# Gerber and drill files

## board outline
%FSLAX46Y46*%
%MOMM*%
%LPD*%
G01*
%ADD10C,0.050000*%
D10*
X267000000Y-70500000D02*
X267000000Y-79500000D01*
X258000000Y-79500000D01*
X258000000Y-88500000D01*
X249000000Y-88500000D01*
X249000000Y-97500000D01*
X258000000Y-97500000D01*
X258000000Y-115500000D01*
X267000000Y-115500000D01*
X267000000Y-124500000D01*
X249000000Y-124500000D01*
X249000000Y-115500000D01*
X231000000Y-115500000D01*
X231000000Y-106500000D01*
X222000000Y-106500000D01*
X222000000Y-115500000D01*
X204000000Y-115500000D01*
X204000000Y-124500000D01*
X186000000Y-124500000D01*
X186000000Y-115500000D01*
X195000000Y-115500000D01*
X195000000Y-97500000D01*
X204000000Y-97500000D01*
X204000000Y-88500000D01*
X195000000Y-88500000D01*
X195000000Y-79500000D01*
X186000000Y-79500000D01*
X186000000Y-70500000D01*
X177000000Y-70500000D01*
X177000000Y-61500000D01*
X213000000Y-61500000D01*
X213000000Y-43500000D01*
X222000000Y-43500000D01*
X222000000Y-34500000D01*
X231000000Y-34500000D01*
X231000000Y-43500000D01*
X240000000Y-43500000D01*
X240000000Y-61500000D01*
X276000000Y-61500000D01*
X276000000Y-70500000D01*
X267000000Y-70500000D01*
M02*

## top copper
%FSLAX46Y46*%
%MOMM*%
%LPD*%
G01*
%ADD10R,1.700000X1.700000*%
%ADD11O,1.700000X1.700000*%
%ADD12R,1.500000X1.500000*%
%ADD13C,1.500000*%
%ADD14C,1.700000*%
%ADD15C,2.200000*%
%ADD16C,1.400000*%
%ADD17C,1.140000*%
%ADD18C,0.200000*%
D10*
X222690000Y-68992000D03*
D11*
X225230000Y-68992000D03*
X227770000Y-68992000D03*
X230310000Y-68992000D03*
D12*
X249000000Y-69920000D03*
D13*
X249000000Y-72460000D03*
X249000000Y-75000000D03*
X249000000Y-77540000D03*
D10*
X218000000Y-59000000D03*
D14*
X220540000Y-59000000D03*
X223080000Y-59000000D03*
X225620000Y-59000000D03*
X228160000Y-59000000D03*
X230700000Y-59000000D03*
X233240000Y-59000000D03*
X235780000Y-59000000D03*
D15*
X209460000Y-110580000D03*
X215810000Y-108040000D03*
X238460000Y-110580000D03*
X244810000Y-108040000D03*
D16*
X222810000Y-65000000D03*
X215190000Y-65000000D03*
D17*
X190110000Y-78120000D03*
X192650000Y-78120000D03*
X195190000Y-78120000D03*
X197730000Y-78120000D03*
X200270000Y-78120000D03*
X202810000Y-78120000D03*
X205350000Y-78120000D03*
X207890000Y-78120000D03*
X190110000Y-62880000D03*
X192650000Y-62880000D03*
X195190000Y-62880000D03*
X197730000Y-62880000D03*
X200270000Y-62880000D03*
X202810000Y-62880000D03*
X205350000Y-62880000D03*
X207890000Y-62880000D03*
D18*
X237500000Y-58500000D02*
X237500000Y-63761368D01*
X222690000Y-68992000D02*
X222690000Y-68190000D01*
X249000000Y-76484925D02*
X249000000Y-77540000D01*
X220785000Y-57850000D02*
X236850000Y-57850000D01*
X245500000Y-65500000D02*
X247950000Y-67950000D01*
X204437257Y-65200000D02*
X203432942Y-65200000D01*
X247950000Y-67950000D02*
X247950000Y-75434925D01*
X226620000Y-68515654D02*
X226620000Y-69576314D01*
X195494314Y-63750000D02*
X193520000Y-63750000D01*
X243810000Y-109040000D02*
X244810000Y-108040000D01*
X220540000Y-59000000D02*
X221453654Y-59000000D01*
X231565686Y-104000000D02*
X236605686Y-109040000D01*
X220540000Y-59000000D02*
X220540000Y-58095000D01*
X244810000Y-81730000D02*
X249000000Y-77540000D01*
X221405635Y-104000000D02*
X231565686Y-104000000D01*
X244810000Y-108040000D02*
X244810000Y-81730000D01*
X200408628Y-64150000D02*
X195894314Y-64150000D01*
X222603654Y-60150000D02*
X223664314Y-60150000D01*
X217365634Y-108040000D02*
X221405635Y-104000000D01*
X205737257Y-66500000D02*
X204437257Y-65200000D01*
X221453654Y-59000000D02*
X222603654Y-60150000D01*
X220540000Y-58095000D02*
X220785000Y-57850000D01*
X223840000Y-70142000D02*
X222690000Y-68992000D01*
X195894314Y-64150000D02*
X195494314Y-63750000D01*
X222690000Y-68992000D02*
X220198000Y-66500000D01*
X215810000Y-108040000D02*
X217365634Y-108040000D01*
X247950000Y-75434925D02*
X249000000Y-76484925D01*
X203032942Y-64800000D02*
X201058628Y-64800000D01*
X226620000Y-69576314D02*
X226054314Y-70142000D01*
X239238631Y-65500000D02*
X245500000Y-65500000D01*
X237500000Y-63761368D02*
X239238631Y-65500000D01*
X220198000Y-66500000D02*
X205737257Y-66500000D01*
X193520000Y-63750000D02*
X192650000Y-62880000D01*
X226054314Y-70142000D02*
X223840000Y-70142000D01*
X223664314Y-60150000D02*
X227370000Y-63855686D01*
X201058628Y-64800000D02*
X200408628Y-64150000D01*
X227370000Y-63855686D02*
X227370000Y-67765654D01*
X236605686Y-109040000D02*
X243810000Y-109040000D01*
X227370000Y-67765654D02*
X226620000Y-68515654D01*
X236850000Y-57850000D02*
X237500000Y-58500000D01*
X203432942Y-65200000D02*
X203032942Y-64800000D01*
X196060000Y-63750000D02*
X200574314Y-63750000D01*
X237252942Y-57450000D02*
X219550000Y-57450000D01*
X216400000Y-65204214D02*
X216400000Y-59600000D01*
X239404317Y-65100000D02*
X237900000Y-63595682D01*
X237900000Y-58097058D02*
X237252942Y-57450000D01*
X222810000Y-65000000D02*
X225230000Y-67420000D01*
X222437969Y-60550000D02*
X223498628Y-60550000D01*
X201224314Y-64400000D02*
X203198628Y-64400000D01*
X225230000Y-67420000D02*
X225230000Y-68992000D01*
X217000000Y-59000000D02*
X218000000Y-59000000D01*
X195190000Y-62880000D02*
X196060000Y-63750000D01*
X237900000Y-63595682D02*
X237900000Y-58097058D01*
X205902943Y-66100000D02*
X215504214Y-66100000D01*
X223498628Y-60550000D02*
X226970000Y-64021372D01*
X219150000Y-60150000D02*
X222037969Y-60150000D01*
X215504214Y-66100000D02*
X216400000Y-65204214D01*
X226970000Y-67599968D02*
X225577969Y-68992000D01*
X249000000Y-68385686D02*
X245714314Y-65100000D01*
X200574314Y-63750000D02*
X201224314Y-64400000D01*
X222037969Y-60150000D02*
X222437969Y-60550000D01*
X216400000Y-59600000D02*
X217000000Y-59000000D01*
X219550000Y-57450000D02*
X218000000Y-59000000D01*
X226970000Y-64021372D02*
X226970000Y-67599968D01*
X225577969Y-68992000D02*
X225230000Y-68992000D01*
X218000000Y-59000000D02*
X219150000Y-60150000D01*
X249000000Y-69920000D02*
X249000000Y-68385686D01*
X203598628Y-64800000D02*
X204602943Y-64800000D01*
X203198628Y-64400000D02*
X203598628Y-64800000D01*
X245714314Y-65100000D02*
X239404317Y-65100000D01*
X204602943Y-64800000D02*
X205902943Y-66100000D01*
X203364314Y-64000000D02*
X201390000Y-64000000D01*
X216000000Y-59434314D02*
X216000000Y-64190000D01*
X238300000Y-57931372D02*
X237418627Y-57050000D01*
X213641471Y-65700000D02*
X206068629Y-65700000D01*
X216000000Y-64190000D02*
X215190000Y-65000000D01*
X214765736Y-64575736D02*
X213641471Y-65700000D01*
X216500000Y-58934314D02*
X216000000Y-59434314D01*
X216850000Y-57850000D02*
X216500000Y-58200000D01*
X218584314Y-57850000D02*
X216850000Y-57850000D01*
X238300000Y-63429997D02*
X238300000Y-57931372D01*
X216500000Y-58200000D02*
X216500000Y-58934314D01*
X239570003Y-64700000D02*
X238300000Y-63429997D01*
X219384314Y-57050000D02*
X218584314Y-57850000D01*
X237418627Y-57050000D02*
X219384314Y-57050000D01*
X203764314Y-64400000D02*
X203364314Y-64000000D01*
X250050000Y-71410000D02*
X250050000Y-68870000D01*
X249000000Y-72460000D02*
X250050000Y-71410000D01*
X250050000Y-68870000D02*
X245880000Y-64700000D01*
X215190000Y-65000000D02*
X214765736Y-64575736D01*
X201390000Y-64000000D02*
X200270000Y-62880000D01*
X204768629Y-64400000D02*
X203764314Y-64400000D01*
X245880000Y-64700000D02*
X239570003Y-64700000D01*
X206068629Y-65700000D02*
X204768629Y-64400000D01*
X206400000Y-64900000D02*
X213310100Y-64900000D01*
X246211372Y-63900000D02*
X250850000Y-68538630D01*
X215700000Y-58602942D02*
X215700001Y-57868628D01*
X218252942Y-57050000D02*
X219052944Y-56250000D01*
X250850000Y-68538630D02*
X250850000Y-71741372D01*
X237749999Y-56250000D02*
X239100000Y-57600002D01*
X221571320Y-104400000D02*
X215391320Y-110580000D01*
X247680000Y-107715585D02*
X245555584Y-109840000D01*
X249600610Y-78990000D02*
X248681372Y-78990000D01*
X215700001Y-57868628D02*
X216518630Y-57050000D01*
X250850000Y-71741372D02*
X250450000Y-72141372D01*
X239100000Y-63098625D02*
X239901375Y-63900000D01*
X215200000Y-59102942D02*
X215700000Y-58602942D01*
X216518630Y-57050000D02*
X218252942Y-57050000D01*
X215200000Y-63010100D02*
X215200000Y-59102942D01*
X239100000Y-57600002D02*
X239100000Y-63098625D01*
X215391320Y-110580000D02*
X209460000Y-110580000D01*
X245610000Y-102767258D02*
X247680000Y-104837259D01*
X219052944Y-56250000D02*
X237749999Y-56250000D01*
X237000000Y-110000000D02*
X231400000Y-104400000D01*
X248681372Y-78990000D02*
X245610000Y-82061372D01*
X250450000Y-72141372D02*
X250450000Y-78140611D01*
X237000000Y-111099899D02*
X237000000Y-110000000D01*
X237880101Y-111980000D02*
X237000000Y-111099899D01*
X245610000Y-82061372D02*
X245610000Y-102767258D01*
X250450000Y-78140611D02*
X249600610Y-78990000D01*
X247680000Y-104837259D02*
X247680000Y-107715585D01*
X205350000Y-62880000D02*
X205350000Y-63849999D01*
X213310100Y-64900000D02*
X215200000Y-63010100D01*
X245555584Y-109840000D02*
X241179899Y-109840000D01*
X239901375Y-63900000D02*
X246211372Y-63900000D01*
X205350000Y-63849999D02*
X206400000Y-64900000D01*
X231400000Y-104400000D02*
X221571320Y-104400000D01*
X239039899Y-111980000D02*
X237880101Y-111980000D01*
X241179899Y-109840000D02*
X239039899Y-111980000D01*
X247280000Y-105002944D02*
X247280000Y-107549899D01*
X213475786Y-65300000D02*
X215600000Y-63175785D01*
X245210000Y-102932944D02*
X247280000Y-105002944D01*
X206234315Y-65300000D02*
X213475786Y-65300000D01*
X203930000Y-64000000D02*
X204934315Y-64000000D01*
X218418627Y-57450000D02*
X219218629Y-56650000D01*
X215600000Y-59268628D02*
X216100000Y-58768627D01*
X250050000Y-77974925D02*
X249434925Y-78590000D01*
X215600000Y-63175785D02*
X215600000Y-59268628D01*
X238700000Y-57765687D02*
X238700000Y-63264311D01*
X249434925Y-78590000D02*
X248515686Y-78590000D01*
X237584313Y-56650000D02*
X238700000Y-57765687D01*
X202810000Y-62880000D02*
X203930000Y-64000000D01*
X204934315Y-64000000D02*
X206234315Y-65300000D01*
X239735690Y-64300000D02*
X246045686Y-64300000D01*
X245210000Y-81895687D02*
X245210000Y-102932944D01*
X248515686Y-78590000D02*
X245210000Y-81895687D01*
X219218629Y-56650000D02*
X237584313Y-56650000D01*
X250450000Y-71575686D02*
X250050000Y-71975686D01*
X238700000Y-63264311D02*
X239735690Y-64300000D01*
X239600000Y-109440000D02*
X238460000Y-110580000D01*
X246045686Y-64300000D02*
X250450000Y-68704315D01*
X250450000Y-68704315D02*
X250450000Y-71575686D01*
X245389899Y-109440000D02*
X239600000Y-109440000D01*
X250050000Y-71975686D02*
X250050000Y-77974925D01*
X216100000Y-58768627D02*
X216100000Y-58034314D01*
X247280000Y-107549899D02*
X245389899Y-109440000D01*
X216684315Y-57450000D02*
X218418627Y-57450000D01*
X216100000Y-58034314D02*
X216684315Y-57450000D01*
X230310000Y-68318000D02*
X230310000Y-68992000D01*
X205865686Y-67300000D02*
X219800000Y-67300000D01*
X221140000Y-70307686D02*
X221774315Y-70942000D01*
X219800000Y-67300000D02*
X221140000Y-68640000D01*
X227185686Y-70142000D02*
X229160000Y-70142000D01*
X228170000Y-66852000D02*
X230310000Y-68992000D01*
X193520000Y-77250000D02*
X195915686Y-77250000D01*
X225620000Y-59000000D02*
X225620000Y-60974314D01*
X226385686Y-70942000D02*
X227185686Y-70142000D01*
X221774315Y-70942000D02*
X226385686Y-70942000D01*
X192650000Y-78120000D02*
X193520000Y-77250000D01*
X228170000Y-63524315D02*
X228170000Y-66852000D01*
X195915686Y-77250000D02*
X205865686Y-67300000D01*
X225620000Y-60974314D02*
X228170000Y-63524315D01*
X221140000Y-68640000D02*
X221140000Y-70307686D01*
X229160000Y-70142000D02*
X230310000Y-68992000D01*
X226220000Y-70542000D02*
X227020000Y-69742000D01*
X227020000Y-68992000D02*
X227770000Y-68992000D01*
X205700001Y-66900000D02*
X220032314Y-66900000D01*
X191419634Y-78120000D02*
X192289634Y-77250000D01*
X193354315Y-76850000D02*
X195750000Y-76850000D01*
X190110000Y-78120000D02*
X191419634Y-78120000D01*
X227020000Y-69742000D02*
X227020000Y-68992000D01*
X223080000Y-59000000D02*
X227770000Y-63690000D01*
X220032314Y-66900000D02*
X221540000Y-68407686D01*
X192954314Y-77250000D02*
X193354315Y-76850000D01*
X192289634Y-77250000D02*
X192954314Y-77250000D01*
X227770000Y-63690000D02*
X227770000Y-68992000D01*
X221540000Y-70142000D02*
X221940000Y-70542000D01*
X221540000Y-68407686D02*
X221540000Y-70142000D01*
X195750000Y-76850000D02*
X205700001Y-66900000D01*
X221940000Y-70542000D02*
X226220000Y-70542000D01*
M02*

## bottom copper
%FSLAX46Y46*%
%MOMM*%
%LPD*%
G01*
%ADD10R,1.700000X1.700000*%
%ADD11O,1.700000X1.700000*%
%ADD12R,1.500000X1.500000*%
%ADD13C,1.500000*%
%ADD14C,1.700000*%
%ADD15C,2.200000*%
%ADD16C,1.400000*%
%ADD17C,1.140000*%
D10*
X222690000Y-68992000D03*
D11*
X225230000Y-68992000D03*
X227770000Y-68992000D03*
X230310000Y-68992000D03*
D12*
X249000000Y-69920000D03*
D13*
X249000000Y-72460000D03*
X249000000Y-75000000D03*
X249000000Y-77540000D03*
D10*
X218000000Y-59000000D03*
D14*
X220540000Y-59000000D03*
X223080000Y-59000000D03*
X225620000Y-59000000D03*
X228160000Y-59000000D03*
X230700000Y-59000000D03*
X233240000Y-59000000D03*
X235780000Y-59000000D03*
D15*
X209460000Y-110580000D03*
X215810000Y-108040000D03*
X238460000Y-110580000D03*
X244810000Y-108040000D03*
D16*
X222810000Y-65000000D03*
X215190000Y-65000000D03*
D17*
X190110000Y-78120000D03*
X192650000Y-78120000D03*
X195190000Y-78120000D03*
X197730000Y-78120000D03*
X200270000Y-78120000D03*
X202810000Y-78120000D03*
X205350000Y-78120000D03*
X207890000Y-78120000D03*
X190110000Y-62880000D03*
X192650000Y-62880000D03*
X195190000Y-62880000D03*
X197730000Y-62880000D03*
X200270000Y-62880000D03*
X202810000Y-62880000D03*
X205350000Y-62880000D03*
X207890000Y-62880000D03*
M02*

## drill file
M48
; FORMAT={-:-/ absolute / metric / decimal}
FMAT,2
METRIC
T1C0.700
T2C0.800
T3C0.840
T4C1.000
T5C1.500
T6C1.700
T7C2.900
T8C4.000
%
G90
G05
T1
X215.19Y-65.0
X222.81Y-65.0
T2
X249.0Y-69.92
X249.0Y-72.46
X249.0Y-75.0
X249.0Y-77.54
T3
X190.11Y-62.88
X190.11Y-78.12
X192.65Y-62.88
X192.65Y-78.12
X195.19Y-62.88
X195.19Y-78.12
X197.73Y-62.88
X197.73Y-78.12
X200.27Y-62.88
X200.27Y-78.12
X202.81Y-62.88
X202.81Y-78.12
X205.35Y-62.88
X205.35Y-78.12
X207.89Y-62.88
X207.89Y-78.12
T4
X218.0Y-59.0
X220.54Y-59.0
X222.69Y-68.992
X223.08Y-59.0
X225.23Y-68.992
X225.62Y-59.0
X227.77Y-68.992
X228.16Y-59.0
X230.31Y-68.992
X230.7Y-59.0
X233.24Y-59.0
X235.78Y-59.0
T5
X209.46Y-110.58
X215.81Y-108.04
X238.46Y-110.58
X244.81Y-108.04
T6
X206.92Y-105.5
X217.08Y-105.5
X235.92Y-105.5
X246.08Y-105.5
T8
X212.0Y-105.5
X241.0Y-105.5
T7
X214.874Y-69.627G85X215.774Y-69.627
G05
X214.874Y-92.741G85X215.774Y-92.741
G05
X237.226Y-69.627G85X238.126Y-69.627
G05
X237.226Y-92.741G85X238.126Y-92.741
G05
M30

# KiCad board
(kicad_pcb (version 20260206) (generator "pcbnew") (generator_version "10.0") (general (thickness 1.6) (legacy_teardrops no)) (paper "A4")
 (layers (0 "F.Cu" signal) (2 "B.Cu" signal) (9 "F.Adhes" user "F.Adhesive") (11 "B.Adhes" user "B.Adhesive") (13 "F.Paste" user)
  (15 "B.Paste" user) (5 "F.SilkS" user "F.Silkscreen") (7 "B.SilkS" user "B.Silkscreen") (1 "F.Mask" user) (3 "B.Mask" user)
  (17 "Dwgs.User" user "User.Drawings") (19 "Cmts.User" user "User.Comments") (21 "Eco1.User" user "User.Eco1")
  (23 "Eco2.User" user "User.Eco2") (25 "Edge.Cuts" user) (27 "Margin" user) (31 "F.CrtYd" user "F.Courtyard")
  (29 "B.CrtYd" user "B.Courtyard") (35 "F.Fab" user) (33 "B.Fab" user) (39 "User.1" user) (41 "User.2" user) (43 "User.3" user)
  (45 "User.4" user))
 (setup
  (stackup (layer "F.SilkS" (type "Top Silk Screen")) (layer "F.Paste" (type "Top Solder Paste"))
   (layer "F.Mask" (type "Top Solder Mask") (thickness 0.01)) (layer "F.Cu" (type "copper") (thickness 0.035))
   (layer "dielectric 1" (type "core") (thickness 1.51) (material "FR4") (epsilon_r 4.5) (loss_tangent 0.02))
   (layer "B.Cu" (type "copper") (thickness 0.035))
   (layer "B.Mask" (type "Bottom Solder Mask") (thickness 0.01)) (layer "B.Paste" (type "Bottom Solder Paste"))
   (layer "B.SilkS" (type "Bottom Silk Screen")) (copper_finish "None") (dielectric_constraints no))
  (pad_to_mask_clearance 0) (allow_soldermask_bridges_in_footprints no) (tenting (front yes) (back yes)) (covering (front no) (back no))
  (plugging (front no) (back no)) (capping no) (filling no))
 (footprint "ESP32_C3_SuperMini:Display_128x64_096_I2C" (layer "F.Cu") (at 226.5 68.992)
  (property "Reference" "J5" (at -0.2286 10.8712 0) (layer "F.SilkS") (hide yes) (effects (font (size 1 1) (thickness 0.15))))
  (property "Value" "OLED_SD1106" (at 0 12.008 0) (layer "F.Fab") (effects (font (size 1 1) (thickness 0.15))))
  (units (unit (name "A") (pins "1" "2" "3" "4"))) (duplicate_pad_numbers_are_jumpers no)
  (pad "" np_thru_hole oval (at -11.176 0.635) (size 3.8 2.9) (drill oval 3.8 2.9) (layers "*.Cu" "*.Mask"))
  (pad "" np_thru_hole oval (at -11.176 23.749) (size 3.8 2.9) (drill oval 3.8 2.9) (layers "*.Cu" "*.Mask"))
  (pad "" np_thru_hole oval (at 11.176 0.635) (size 3.8 2.9) (drill oval 3.8 2.9) (layers "*.Cu" "*.Mask"))
  (pad "" np_thru_hole oval (at 11.176 23.749) (size 3.8 2.9) (drill oval 3.8 2.9) (layers "*.Cu" "*.Mask"))
  (pad "1" thru_hole rect (at -3.81 0 90) (size 1.7 1.7) (drill 1) (layers "*.Cu" "*.Mask") (remove_unused_layers no) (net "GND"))
  (pad "2" thru_hole oval (at -1.27 0 90) (size 1.7 1.7) (drill 1) (layers "*.Cu" "*.Mask") (remove_unused_layers no) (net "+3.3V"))
  (pad "3" thru_hole oval (at 1.27 0 90) (size 1.7 1.7) (drill 1) (layers "*.Cu" "*.Mask") (remove_unused_layers no) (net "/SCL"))
  (pad "4" thru_hole oval (at 3.81 0 90) (size 1.7 1.7) (drill 1) (layers "*.Cu" "*.Mask") (remove_unused_layers no) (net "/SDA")))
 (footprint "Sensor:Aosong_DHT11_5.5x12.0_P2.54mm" (layer "F.Cu") (at 249 69.92)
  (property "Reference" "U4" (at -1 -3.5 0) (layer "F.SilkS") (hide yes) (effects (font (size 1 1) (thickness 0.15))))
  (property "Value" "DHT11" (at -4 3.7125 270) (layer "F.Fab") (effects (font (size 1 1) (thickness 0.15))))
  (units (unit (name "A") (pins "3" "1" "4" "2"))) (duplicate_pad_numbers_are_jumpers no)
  (pad "1" thru_hole rect (at 0 0) (size 1.5 1.5) (drill 0.8) (layers "*.Cu" "*.Mask") (remove_unused_layers no) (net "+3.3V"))
  (pad "2" thru_hole circle (at 0 2.54) (size 1.5 1.5) (drill 0.8) (layers "*.Cu" "*.Mask") (remove_unused_layers no) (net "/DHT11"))
  (pad "3" thru_hole circle (at 0 5.08) (size 1.5 1.5) (drill 0.8) (layers "*.Cu" "*.Mask") (remove_unused_layers no)
   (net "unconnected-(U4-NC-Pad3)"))
  (pad "4" thru_hole circle (at 0 7.62) (size 1.5 1.5) (drill 0.8) (layers "*.Cu" "*.Mask") (remove_unused_layers no) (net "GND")))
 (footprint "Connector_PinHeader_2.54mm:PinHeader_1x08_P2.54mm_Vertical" (layer "F.Cu") (at 218 59 90)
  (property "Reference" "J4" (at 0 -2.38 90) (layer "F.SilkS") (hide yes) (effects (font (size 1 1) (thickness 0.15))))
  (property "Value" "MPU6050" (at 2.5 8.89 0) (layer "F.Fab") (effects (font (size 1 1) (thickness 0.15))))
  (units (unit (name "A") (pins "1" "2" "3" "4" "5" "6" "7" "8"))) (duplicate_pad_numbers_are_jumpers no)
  (pad "1" thru_hole rect (at 0 0 90) (size 1.7 1.7) (drill 1) (layers "*.Cu" "*.Mask") (remove_unused_layers no) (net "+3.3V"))
  (pad "2" thru_hole circle (at 0 2.54 90) (size 1.7 1.7) (drill 1) (layers "*.Cu" "*.Mask") (remove_unused_layers no) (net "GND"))
  (pad "3" thru_hole circle (at 0 5.08 90) (size 1.7 1.7) (drill 1) (layers "*.Cu" "*.Mask") (remove_unused_layers no) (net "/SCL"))
  (pad "4" thru_hole circle (at 0 7.62 90) (size 1.7 1.7) (drill 1) (layers "*.Cu" "*.Mask") (remove_unused_layers no) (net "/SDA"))
  (pad "5" thru_hole circle (at 0 10.16 90) (size 1.7 1.7) (drill 1) (layers "*.Cu" "*.Mask") (remove_unused_layers no)
   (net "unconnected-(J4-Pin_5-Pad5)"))
  (pad "6" thru_hole circle (at 0 12.7 90) (size 1.7 1.7) (drill 1) (layers "*.Cu" "*.Mask") (remove_unused_layers no)
   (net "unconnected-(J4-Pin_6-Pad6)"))
  (pad "7" thru_hole circle (at 0 15.24 90) (size 1.7 1.7) (drill 1) (layers "*.Cu" "*.Mask") (remove_unused_layers no)
   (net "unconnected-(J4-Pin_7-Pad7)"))
  (pad "8" thru_hole circle (at 0 17.78 90) (size 1.7 1.7) (drill 1) (layers "*.Cu" "*.Mask") (remove_unused_layers no)
   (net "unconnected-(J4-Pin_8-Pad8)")))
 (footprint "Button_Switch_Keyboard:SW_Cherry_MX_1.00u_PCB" (layer "F.Cu") (at 209.46 110.58 180)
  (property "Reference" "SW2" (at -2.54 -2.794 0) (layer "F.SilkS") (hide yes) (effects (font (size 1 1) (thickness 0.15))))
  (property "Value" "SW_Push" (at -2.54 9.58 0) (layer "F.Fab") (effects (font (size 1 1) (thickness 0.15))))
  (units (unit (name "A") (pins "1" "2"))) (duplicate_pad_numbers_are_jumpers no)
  (pad "" np_thru_hole circle (at -7.62 5.08 180) (size 1.7 1.7) (drill 1.7) (layers "*.Cu" "*.Mask"))
  (pad "" np_thru_hole circle (at -2.54 5.08 180) (size 4 4) (drill 4) (layers "*.Cu" "*.Mask"))
  (pad "" np_thru_hole circle (at 2.54 5.08 180) (size 1.7 1.7) (drill 1.7) (layers "*.Cu" "*.Mask"))
  (pad "1" thru_hole circle (at 0 0 180) (size 2.2 2.2) (drill 1.5) (layers "*.Cu" "*.Mask") (remove_unused_layers no) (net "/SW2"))
  (pad "2" thru_hole circle (at -6.35 2.54 180) (size 2.2 2.2) (drill 1.5) (layers "*.Cu" "*.Mask") (remove_unused_layers no) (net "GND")))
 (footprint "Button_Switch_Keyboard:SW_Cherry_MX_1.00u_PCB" (layer "F.Cu") (at 238.46 110.58 180)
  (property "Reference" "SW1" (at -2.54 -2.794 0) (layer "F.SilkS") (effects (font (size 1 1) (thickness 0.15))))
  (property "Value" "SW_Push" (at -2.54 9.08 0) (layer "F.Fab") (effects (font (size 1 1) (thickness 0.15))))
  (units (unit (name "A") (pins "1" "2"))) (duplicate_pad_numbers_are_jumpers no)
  (pad "" np_thru_hole circle (at -7.62 5.08 180) (size 1.7 1.7) (drill 1.7) (layers "*.Cu" "*.Mask"))
  (pad "" np_thru_hole circle (at -2.54 5.08 180) (size 4 4) (drill 4) (layers "*.Cu" "*.Mask"))
  (pad "" np_thru_hole circle (at 2.54 5.08 180) (size 1.7 1.7) (drill 1.7) (layers "*.Cu" "*.Mask"))
  (pad "1" thru_hole circle (at 0 0 180) (size 2.2 2.2) (drill 1.5) (layers "*.Cu" "*.Mask") (remove_unused_layers no) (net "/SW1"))
  (pad "2" thru_hole circle (at -6.35 2.54 180) (size 2.2 2.2) (drill 1.5) (layers "*.Cu" "*.Mask") (remove_unused_layers no) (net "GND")))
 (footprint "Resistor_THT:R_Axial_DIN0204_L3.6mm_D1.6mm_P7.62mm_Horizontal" (layer "F.Cu") (at 222.81 65 180)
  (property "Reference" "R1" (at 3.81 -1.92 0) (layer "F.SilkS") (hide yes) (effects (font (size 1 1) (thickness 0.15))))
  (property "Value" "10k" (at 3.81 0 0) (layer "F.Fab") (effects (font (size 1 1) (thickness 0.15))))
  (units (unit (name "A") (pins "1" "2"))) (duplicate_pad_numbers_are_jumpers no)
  (pad "1" thru_hole circle (at 0 0 180) (size 1.4 1.4) (drill 0.7) (layers "*.Cu" "*.Mask") (remove_unused_layers no) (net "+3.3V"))
  (pad "2" thru_hole circle (at 7.62 0 180) (size 1.4 1.4) (drill 0.7) (layers "*.Cu" "*.Mask") (remove_unused_layers no) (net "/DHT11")))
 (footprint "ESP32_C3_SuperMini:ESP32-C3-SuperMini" (layer "F.Cu") (at 199 70.5 90)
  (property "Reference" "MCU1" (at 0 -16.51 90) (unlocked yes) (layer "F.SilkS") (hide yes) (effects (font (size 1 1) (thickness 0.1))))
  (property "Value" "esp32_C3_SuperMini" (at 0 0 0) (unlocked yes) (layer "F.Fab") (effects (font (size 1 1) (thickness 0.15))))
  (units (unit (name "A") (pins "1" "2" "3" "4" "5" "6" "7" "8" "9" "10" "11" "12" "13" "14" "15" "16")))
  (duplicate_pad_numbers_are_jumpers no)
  (pad "1" thru_hole circle (at -7.62 -8.89 90) (size 1.14 1.14) (drill 0.84) (layers "*.Cu" "*.Mask") (remove_unused_layers no)
   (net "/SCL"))
  (pad "2" thru_hole circle (at -7.62 -6.35 90) (size 1.14 1.14) (drill 0.84) (layers "*.Cu" "*.Mask") (remove_unused_layers no)
   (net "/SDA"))
  (pad "3" thru_hole circle (at -7.62 -3.81 90) (size 1.14 1.14) (drill 0.84) (layers "*.Cu" "*.Mask") (remove_unused_layers no)
   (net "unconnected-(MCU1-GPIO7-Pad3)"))
  (pad "4" thru_hole circle (at -7.62 -1.27 90) (size 1.14 1.14) (drill 0.84) (layers "*.Cu" "*.Mask") (remove_unused_layers no)
   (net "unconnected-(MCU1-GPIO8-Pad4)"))
  (pad "5" thru_hole circle (at -7.62 1.27 90) (size 1.14 1.14) (drill 0.84) (layers "*.Cu" "*.Mask") (remove_unused_layers no)
   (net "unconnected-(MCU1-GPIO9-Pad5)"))
  (pad "6" thru_hole circle (at -7.62 3.81 90) (size 1.14 1.14) (drill 0.84) (layers "*.Cu" "*.Mask") (remove_unused_layers no)
   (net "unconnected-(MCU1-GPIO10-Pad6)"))
  (pad "7" thru_hole circle (at -7.62 6.35 90) (size 1.14 1.14) (drill 0.84) (layers "*.Cu" "*.Mask") (remove_unused_layers no)
   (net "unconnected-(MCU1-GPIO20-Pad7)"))
  (pad "8" thru_hole circle (at -7.62 8.89 90) (size 1.14 1.14) (drill 0.84) (layers "*.Cu" "*.Mask") (remove_unused_layers no)
   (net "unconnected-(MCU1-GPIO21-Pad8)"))
  (pad "9" thru_hole circle (at 7.62 -8.89 90) (size 1.14 1.14) (drill 0.84) (layers "*.Cu" "*.Mask") (remove_unused_layers no)
   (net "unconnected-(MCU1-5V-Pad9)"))
  (pad "10" thru_hole circle (at 7.62 -6.35 90) (size 1.14 1.14) (drill 0.84) (layers "*.Cu" "*.Mask") (remove_unused_layers no) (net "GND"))
  (pad "11" thru_hole circle (at 7.62 -3.81 90) (size 1.14 1.14) (drill 0.84) (layers "*.Cu" "*.Mask") (remove_unused_layers no)
   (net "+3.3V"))
  (pad "12" thru_hole circle (at 7.62 -1.27 90) (size 1.14 1.14) (drill 0.84) (layers "*.Cu" "*.Mask") (remove_unused_layers no)
   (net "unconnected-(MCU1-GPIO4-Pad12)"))
  (pad "13" thru_hole circle (at 7.62 1.27 90) (size 1.14 1.14) (drill 0.84) (layers "*.Cu" "*.Mask") (remove_unused_layers no)
   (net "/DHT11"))
  (pad "14" thru_hole circle (at 7.62 3.81 90) (size 1.14 1.14) (drill 0.84) (layers "*.Cu" "*.Mask") (remove_unused_layers no) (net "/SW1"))
  (pad "15" thru_hole circle (at 7.62 6.35 90) (size 1.14 1.14) (drill 0.84) (layers "*.Cu" "*.Mask") (remove_unused_layers no) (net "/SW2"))
  (pad "16" thru_hole circle (at 7.62 8.89 90) (size 1.14 1.14) (drill 0.84) (layers "*.Cu" "*.Mask") (remove_unused_layers no)
   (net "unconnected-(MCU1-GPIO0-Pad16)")))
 (gr_poly
  (pts (xy 267 70.5) (xy 267 79.5) (xy 258 79.5) (xy 258 88.5) (xy 249 88.5) (xy 249 97.5) (xy 258 97.5) (xy 258 115.5) (xy 267 115.5)
   (xy 267 124.5) (xy 249 124.5) (xy 249 115.5) (xy 231 115.5) (xy 231 106.5) (xy 222 106.5) (xy 222 115.5) (xy 204 115.5) (xy 204 124.5)
   (xy 186 124.5) (xy 186 115.5) (xy 195 115.5) (xy 195 97.5) (xy 204 97.5) (xy 204 88.5) (xy 195 88.5) (xy 195 79.5) (xy 186 79.5)
   (xy 186 70.5) (xy 177 70.5) (xy 177 61.5) (xy 213 61.5) (xy 213 43.5) (xy 222 43.5) (xy 222 34.5) (xy 231 34.5) (xy 231 43.5)
   (xy 240 43.5) (xy 240 61.5) (xy 276 61.5) (xy 276 70.5))
  (stroke (width 0.05) (type solid)) (fill no) (layer "Edge.Cuts"))
 (segment (start 237.5 58.5) (end 237.5 63.761368) (width 0.2) (layer "F.Cu") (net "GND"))
 (segment (start 222.69 68.992) (end 222.69 68.19) (width 0.2) (layer "F.Cu") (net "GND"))
 (segment (start 249 76.484925) (end 249 77.54) (width 0.2) (layer "F.Cu") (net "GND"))
 (segment (start 220.785 57.85) (end 236.85 57.85) (width 0.2) (layer "F.Cu") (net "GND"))
 (segment (start 245.5 65.5) (end 247.95 67.95) (width 0.2) (layer "F.Cu") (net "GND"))
 (segment (start 204.437257 65.2) (end 203.432942 65.2) (width 0.2) (layer "F.Cu") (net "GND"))
 (segment (start 247.95 67.95) (end 247.95 75.434925) (width 0.2) (layer "F.Cu") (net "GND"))
 (segment (start 226.62 68.515654) (end 226.62 69.576314) (width 0.2) (layer "F.Cu") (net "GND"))
 (segment (start 195.494314 63.75) (end 193.52 63.75) (width 0.2) (layer "F.Cu") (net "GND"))
 (segment (start 243.81 109.04) (end 244.81 108.04) (width 0.2) (layer "F.Cu") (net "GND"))
 (segment (start 220.54 59) (end 221.453654 59) (width 0.2) (layer "F.Cu") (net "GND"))
 (segment (start 231.565686 104) (end 236.605686 109.04) (width 0.2) (layer "F.Cu") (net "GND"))
 (segment (start 220.54 59) (end 220.54 58.095) (width 0.2) (layer "F.Cu") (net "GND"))
 (segment (start 244.81 81.73) (end 249 77.54) (width 0.2) (layer "F.Cu") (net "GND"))
 (segment (start 221.405635 104) (end 231.565686 104) (width 0.2) (layer "F.Cu") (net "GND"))
 (segment (start 244.81 108.04) (end 244.81 81.73) (width 0.2) (layer "F.Cu") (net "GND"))
 (segment (start 200.408628 64.15) (end 195.894314 64.15) (width 0.2) (layer "F.Cu") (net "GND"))
 (segment (start 222.603654 60.15) (end 223.664314 60.15) (width 0.2) (layer "F.Cu") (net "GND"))
 (segment (start 217.365634 108.04) (end 221.405635 104) (width 0.2) (layer "F.Cu") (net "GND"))
 (segment (start 205.737257 66.5) (end 204.437257 65.2) (width 0.2) (layer "F.Cu") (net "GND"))
 (segment (start 221.453654 59) (end 222.603654 60.15) (width 0.2) (layer "F.Cu") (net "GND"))
 (segment (start 220.54 58.095) (end 220.785 57.85) (width 0.2) (layer "F.Cu") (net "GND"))
 (segment (start 223.84 70.142) (end 222.69 68.992) (width 0.2) (layer "F.Cu") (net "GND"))
 (segment (start 195.894314 64.15) (end 195.494314 63.75) (width 0.2) (layer "F.Cu") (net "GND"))
 (segment (start 222.69 68.992) (end 220.198 66.5) (width 0.2) (layer "F.Cu") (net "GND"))
 (segment (start 215.81 108.04) (end 217.365634 108.04) (width 0.2) (layer "F.Cu") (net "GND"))
 (segment (start 247.95 75.434925) (end 249 76.484925) (width 0.2) (layer "F.Cu") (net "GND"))
 (segment (start 203.032942 64.8) (end 201.058628 64.8) (width 0.2) (layer "F.Cu") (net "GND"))
 (segment (start 226.62 69.576314) (end 226.054314 70.142) (width 0.2) (layer "F.Cu") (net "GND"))
 (segment (start 239.238631 65.5) (end 245.5 65.5) (width 0.2) (layer "F.Cu") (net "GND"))
 (segment (start 237.5 63.761368) (end 239.238631 65.5) (width 0.2) (layer "F.Cu") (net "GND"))
 (segment (start 220.198 66.5) (end 205.737257 66.5) (width 0.2) (layer "F.Cu") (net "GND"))
 (segment (start 193.52 63.75) (end 192.65 62.88) (width 0.2) (layer "F.Cu") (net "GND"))
 (segment (start 226.054314 70.142) (end 223.84 70.142) (width 0.2) (layer "F.Cu") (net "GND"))
 (segment (start 223.664314 60.15) (end 227.37 63.855686) (width 0.2) (layer "F.Cu") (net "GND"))
 (segment (start 201.058628 64.8) (end 200.408628 64.15) (width 0.2) (layer "F.Cu") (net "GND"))
 (segment (start 227.37 63.855686) (end 227.37 67.765654) (width 0.2) (layer "F.Cu") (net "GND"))
 (segment (start 236.605686 109.04) (end 243.81 109.04) (width 0.2) (layer "F.Cu") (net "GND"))
 (segment (start 227.37 67.765654) (end 226.62 68.515654) (width 0.2) (layer "F.Cu") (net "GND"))
 (segment (start 236.85 57.85) (end 237.5 58.5) (width 0.2) (layer "F.Cu") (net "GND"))
 (segment (start 203.432942 65.2) (end 203.032942 64.8) (width 0.2) (layer "F.Cu") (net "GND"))
 (segment (start 196.06 63.75) (end 200.574314 63.75) (width 0.2) (layer "F.Cu") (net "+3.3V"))
 (segment (start 237.252942 57.45) (end 219.55 57.45) (width 0.2) (layer "F.Cu") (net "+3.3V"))
 (segment (start 216.4 65.204214) (end 216.4 59.6) (width 0.2) (layer "F.Cu") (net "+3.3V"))
 (segment (start 239.404317 65.1) (end 237.9 63.595682) (width 0.2) (layer "F.Cu") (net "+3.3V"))
 (segment (start 237.9 58.097058) (end 237.252942 57.45) (width 0.2) (layer "F.Cu") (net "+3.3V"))
 (segment (start 222.81 65) (end 225.23 67.42) (width 0.2) (layer "F.Cu") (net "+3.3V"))
 (segment (start 222.437969 60.55) (end 223.498628 60.55) (width 0.2) (layer "F.Cu") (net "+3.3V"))
 (segment (start 201.224314 64.4) (end 203.198628 64.4) (width 0.2) (layer "F.Cu") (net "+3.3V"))
 (segment (start 225.23 67.42) (end 225.23 68.992) (width 0.2) (layer "F.Cu") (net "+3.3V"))
 (segment (start 217 59) (end 218 59) (width 0.2) (layer "F.Cu") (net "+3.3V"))
 (segment (start 195.19 62.88) (end 196.06 63.75) (width 0.2) (layer "F.Cu") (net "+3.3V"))
 (segment (start 237.9 63.595682) (end 237.9 58.097058) (width 0.2) (layer "F.Cu") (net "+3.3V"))
 (segment (start 205.902943 66.1) (end 215.504214 66.1) (width 0.2) (layer "F.Cu") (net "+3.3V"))
 (segment (start 223.498628 60.55) (end 226.97 64.021372) (width 0.2) (layer "F.Cu") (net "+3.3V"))
 (segment (start 219.15 60.15) (end 222.037969 60.15) (width 0.2) (layer "F.Cu") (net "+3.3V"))
 (segment (start 215.504214 66.1) (end 216.4 65.204214) (width 0.2) (layer "F.Cu") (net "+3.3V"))
 (segment (start 226.97 67.599968) (end 225.577969 68.992) (width 0.2) (layer "F.Cu") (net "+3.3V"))
 (segment (start 249 68.385686) (end 245.714314 65.1) (width 0.2) (layer "F.Cu") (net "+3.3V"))
 (segment (start 200.574314 63.75) (end 201.224314 64.4) (width 0.2) (layer "F.Cu") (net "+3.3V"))
 (segment (start 222.037969 60.15) (end 222.437969 60.55) (width 0.2) (layer "F.Cu") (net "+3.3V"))
 (segment (start 216.4 59.6) (end 217 59) (width 0.2) (layer "F.Cu") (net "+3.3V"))
 (segment (start 219.55 57.45) (end 218 59) (width 0.2) (layer "F.Cu") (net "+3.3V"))
 (segment (start 226.97 64.021372) (end 226.97 67.599968) (width 0.2) (layer "F.Cu") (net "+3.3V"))
 (segment (start 225.577969 68.992) (end 225.23 68.992) (width 0.2) (layer "F.Cu") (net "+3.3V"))
 (segment (start 218 59) (end 219.15 60.15) (width 0.2) (layer "F.Cu") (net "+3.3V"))
 (segment (start 249 69.92) (end 249 68.385686) (width 0.2) (layer "F.Cu") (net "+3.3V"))
 (segment (start 203.598628 64.8) (end 204.602943 64.8) (width 0.2) (layer "F.Cu") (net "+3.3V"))
 (segment (start 203.198628 64.4) (end 203.598628 64.8) (width 0.2) (layer "F.Cu") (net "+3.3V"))
 (segment (start 245.714314 65.1) (end 239.404317 65.1) (width 0.2) (layer "F.Cu") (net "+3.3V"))
 (segment (start 204.602943 64.8) (end 205.902943 66.1) (width 0.2) (layer "F.Cu") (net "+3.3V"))
 (segment (start 203.364314 64) (end 201.39 64) (width 0.2) (layer "F.Cu") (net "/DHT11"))
 (segment (start 216 59.434314) (end 216 64.19) (width 0.2) (layer "F.Cu") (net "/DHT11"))
 (segment (start 238.3 57.931372) (end 237.418627 57.05) (width 0.2) (layer "F.Cu") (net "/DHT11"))
 (segment (start 213.641471 65.7) (end 206.068629 65.7) (width 0.2) (layer "F.Cu") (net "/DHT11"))
 (segment (start 216 64.19) (end 215.19 65) (width 0.2) (layer "F.Cu") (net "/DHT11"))
 (segment (start 214.765736 64.575736) (end 213.641471 65.7) (width 0.2) (layer "F.Cu") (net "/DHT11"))
 (segment (start 216.5 58.934314) (end 216 59.434314) (width 0.2) (layer "F.Cu") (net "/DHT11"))
 (segment (start 216.85 57.85) (end 216.5 58.2) (width 0.2) (layer "F.Cu") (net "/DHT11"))
 (segment (start 218.584314 57.85) (end 216.85 57.85) (width 0.2) (layer "F.Cu") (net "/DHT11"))
 (segment (start 238.3 63.429997) (end 238.3 57.931372) (width 0.2) (layer "F.Cu") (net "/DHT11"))
 (segment (start 216.5 58.2) (end 216.5 58.934314) (width 0.2) (layer "F.Cu") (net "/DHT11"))
 (segment (start 239.570003 64.7) (end 238.3 63.429997) (width 0.2) (layer "F.Cu") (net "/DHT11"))
 (segment (start 219.384314 57.05) (end 218.584314 57.85) (width 0.2) (layer "F.Cu") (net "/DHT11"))
 (segment (start 237.418627 57.05) (end 219.384314 57.05) (width 0.2) (layer "F.Cu") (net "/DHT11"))
 (segment (start 203.764314 64.4) (end 203.364314 64) (width 0.2) (layer "F.Cu") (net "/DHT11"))
 (segment (start 250.05 71.41) (end 250.05 68.87) (width 0.2) (layer "F.Cu") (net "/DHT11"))
 (segment (start 249 72.46) (end 250.05 71.41) (width 0.2) (layer "F.Cu") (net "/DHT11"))
 (segment (start 250.05 68.87) (end 245.88 64.7) (width 0.2) (layer "F.Cu") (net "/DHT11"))
 (segment (start 215.19 65) (end 214.765736 64.575736) (width 0.2) (layer "F.Cu") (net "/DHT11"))
 (segment (start 201.39 64) (end 200.27 62.88) (width 0.2) (layer "F.Cu") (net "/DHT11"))
 (segment (start 204.768629 64.4) (end 203.764314 64.4) (width 0.2) (layer "F.Cu") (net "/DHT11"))
 (segment (start 245.88 64.7) (end 239.570003 64.7) (width 0.2) (layer "F.Cu") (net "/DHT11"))
 (segment (start 206.068629 65.7) (end 204.768629 64.4) (width 0.2) (layer "F.Cu") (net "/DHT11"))
 (segment (start 206.4 64.9) (end 213.3101 64.9) (width 0.2) (layer "F.Cu") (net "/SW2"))
 (segment (start 246.211372 63.9) (end 250.85 68.53863) (width 0.2) (layer "F.Cu") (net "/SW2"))
 (segment (start 215.7 58.602942) (end 215.700001 57.868628) (width 0.2) (layer "F.Cu") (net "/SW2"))
 (segment (start 218.252942 57.05) (end 219.052944 56.25) (width 0.2) (layer "F.Cu") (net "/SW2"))
 (segment (start 250.85 68.53863) (end 250.85 71.741372) (width 0.2) (layer "F.Cu") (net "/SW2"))
 (segment (start 237.749999 56.25) (end 239.1 57.600002) (width 0.2) (layer "F.Cu") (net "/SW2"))
 (segment (start 221.57132 104.4) (end 215.39132 110.58) (width 0.2) (layer "F.Cu") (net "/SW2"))
 (segment (start 247.68 107.715585) (end 245.555584 109.84) (width 0.2) (layer "F.Cu") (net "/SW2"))
 (segment (start 249.60061 78.99) (end 248.681372 78.99) (width 0.2) (layer "F.Cu") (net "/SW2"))
 (segment (start 215.700001 57.868628) (end 216.51863 57.05) (width 0.2) (layer "F.Cu") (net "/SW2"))
 (segment (start 250.85 71.741372) (end 250.45 72.141372) (width 0.2) (layer "F.Cu") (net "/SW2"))
 (segment (start 239.1 63.098625) (end 239.901375 63.9) (width 0.2) (layer "F.Cu") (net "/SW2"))
 (segment (start 215.2 59.102942) (end 215.7 58.602942) (width 0.2) (layer "F.Cu") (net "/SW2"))
 (segment (start 216.51863 57.05) (end 218.252942 57.05) (width 0.2) (layer "F.Cu") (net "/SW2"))
 (segment (start 215.2 63.0101) (end 215.2 59.102942) (width 0.2) (layer "F.Cu") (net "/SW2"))
 (segment (start 239.1 57.600002) (end 239.1 63.098625) (width 0.2) (layer "F.Cu") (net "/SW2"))
 (segment (start 215.39132 110.58) (end 209.46 110.58) (width 0.2) (layer "F.Cu") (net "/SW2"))
 (segment (start 245.61 102.767258) (end 247.68 104.837259) (width 0.2) (layer "F.Cu") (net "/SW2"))
 (segment (start 219.052944 56.25) (end 237.749999 56.25) (width 0.2) (layer "F.Cu") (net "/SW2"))
 (segment (start 237 110) (end 231.4 104.4) (width 0.2) (layer "F.Cu") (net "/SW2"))
 (segment (start 248.681372 78.99) (end 245.61 82.061372) (width 0.2) (layer "F.Cu") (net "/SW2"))
 (segment (start 250.45 72.141372) (end 250.45 78.140611) (width 0.2) (layer "F.Cu") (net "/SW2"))
 (segment (start 237 111.099899) (end 237 110) (width 0.2) (layer "F.Cu") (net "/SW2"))
 (segment (start 237.880101 111.98) (end 237 111.099899) (width 0.2) (layer "F.Cu") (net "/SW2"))
 (segment (start 245.61 82.061372) (end 245.61 102.767258) (width 0.2) (layer "F.Cu") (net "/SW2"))
 (segment (start 250.45 78.140611) (end 249.60061 78.99) (width 0.2) (layer "F.Cu") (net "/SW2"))
 (segment (start 247.68 104.837259) (end 247.68 107.715585) (width 0.2) (layer "F.Cu") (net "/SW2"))
 (segment (start 205.35 62.88) (end 205.35 63.849999) (width 0.2) (layer "F.Cu") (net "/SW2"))
 (segment (start 213.3101 64.9) (end 215.2 63.0101) (width 0.2) (layer "F.Cu") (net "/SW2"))
 (segment (start 245.555584 109.84) (end 241.179899 109.84) (width 0.2) (layer "F.Cu") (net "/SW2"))
 (segment (start 239.901375 63.9) (end 246.211372 63.9) (width 0.2) (layer "F.Cu") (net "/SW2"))
 (segment (start 205.35 63.849999) (end 206.4 64.9) (width 0.2) (layer "F.Cu") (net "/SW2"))
 (segment (start 231.4 104.4) (end 221.57132 104.4) (width 0.2) (layer "F.Cu") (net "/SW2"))
 (segment (start 239.039899 111.98) (end 237.880101 111.98) (width 0.2) (layer "F.Cu") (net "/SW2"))
 (segment (start 241.179899 109.84) (end 239.039899 111.98) (width 0.2) (layer "F.Cu") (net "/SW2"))
 (segment (start 247.28 105.002944) (end 247.28 107.549899) (width 0.2) (layer "F.Cu") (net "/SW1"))
 (segment (start 213.475786 65.3) (end 215.6 63.175785) (width 0.2) (layer "F.Cu") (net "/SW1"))
 (segment (start 245.21 102.932944) (end 247.28 105.002944) (width 0.2) (layer "F.Cu") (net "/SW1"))
 (segment (start 206.234315 65.3) (end 213.475786 65.3) (width 0.2) (layer "F.Cu") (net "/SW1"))
 (segment (start 203.93 64) (end 204.934315 64) (width 0.2) (layer "F.Cu") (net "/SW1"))
 (segment (start 218.418627 57.45) (end 219.218629 56.65) (width 0.2) (layer "F.Cu") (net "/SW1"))
 (segment (start 215.6 59.268628) (end 216.1 58.768627) (width 0.2) (layer "F.Cu") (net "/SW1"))
 (segment (start 250.05 77.974925) (end 249.434925 78.59) (width 0.2) (layer "F.Cu") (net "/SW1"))
 (segment (start 215.6 63.175785) (end 215.6 59.268628) (width 0.2) (layer "F.Cu") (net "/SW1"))
 (segment (start 238.7 57.765687) (end 238.7 63.264311) (width 0.2) (layer "F.Cu") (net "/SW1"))
 (segment (start 249.434925 78.59) (end 248.515686 78.59) (width 0.2) (layer "F.Cu") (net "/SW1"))
 (segment (start 237.584313 56.65) (end 238.7 57.765687) (width 0.2) (layer "F.Cu") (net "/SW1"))
 (segment (start 202.81 62.88) (end 203.93 64) (width 0.2) (layer "F.Cu") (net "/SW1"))
 (segment (start 204.934315 64) (end 206.234315 65.3) (width 0.2) (layer "F.Cu") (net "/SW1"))
 (segment (start 239.73569 64.3) (end 246.045686 64.3) (width 0.2) (layer "F.Cu") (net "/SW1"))
 (segment (start 245.21 81.895687) (end 245.21 102.932944) (width 0.2) (layer "F.Cu") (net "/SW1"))
 (segment (start 248.515686 78.59) (end 245.21 81.895687) (width 0.2) (layer "F.Cu") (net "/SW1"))
 (segment (start 219.218629 56.65) (end 237.584313 56.65) (width 0.2) (layer "F.Cu") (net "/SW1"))
 (segment (start 250.45 71.575686) (end 250.05 71.975686) (width 0.2) (layer "F.Cu") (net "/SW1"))
 (segment (start 238.7 63.264311) (end 239.73569 64.3) (width 0.2) (layer "F.Cu") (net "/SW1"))
 (segment (start 239.6 109.44) (end 238.46 110.58) (width 0.2) (layer "F.Cu") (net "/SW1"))
 (segment (start 246.045686 64.3) (end 250.45 68.704315) (width 0.2) (layer "F.Cu") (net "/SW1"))
 (segment (start 250.45 68.704315) (end 250.45 71.575686) (width 0.2) (layer "F.Cu") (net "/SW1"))
 (segment (start 245.389899 109.44) (end 239.6 109.44) (width 0.2) (layer "F.Cu") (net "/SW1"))
 (segment (start 250.05 71.975686) (end 250.05 77.974925) (width 0.2) (layer "F.Cu") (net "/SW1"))
 (segment (start 216.1 58.768627) (end 216.1 58.034314) (width 0.2) (layer "F.Cu") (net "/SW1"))
 (segment (start 247.28 107.549899) (end 245.389899 109.44) (width 0.2) (layer "F.Cu") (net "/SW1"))
 (segment (start 216.684315 57.45) (end 218.418627 57.45) (width 0.2) (layer "F.Cu") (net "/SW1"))
 (segment (start 216.1 58.034314) (end 216.684315 57.45) (width 0.2) (layer "F.Cu") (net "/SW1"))
 (segment (start 230.31 68.318) (end 230.31 68.992) (width 0.2) (layer "F.Cu") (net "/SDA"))
 (segment (start 205.865686 67.3) (end 219.8 67.3) (width 0.2) (layer "F.Cu") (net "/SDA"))
 (segment (start 221.14 70.307686) (end 221.774315 70.942) (width 0.2) (layer "F.Cu") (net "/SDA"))
 (segment (start 219.8 67.3) (end 221.14 68.64) (width 0.2) (layer "F.Cu") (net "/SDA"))
 (segment (start 227.185686 70.142) (end 229.16 70.142) (width 0.2) (layer "F.Cu") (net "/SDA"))
 (segment (start 228.17 66.852) (end 230.31 68.992) (width 0.2) (layer "F.Cu") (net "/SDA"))
 (segment (start 193.52 77.25) (end 195.915686 77.25) (width 0.2) (layer "F.Cu") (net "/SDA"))
 (segment (start 225.62 59) (end 225.62 60.974314) (width 0.2) (layer "F.Cu") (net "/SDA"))
 (segment (start 226.385686 70.942) (end 227.185686 70.142) (width 0.2) (layer "F.Cu") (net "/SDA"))
 (segment (start 221.774315 70.942) (end 226.385686 70.942) (width 0.2) (layer "F.Cu") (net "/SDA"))
 (segment (start 192.65 78.12) (end 193.52 77.25) (width 0.2) (layer "F.Cu") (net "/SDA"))
 (segment (start 228.17 63.524315) (end 228.17 66.852) (width 0.2) (layer "F.Cu") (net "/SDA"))
 (segment (start 195.915686 77.25) (end 205.865686 67.3) (width 0.2) (layer "F.Cu") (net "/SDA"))
 (segment (start 225.62 60.974314) (end 228.17 63.524315) (width 0.2) (layer "F.Cu") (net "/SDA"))
 (segment (start 221.14 68.64) (end 221.14 70.307686) (width 0.2) (layer "F.Cu") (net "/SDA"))
 (segment (start 229.16 70.142) (end 230.31 68.992) (width 0.2) (layer "F.Cu") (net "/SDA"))
 (segment (start 226.22 70.542) (end 227.02 69.742) (width 0.2) (layer "F.Cu") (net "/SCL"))
 (segment (start 227.02 68.992) (end 227.77 68.992) (width 0.2) (layer "F.Cu") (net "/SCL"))
 (segment (start 205.700001 66.9) (end 220.032314 66.9) (width 0.2) (layer "F.Cu") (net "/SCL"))
 (segment (start 191.419634 78.12) (end 192.289634 77.25) (width 0.2) (layer "F.Cu") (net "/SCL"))
 (segment (start 193.354315 76.85) (end 195.75 76.85) (width 0.2) (layer "F.Cu") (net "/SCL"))
 (segment (start 190.11 78.12) (end 191.419634 78.12) (width 0.2) (layer "F.Cu") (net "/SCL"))
 (segment (start 227.02 69.742) (end 227.02 68.992) (width 0.2) (layer "F.Cu") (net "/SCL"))
 (segment (start 223.08 59) (end 227.77 63.69) (width 0.2) (layer "F.Cu") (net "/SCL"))
 (segment (start 220.032314 66.9) (end 221.54 68.407686) (width 0.2) (layer "F.Cu") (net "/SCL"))
 (segment (start 192.954314 77.25) (end 193.354315 76.85) (width 0.2) (layer "F.Cu") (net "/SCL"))
 (segment (start 192.289634 77.25) (end 192.954314 77.25) (width 0.2) (layer "F.Cu") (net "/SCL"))
 (segment (start 227.77 63.69) (end 227.77 68.992) (width 0.2) (layer "F.Cu") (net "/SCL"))
 (segment (start 221.54 70.142) (end 221.94 70.542) (width 0.2) (layer "F.Cu") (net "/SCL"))
 (segment (start 221.54 68.407686) (end 221.54 70.142) (width 0.2) (layer "F.Cu") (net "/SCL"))
 (segment (start 195.75 76.85) (end 205.700001 66.9) (width 0.2) (layer "F.Cu") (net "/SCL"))
 (segment (start 221.94 70.542) (end 226.22 70.542) (width 0.2) (layer "F.Cu") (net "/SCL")))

